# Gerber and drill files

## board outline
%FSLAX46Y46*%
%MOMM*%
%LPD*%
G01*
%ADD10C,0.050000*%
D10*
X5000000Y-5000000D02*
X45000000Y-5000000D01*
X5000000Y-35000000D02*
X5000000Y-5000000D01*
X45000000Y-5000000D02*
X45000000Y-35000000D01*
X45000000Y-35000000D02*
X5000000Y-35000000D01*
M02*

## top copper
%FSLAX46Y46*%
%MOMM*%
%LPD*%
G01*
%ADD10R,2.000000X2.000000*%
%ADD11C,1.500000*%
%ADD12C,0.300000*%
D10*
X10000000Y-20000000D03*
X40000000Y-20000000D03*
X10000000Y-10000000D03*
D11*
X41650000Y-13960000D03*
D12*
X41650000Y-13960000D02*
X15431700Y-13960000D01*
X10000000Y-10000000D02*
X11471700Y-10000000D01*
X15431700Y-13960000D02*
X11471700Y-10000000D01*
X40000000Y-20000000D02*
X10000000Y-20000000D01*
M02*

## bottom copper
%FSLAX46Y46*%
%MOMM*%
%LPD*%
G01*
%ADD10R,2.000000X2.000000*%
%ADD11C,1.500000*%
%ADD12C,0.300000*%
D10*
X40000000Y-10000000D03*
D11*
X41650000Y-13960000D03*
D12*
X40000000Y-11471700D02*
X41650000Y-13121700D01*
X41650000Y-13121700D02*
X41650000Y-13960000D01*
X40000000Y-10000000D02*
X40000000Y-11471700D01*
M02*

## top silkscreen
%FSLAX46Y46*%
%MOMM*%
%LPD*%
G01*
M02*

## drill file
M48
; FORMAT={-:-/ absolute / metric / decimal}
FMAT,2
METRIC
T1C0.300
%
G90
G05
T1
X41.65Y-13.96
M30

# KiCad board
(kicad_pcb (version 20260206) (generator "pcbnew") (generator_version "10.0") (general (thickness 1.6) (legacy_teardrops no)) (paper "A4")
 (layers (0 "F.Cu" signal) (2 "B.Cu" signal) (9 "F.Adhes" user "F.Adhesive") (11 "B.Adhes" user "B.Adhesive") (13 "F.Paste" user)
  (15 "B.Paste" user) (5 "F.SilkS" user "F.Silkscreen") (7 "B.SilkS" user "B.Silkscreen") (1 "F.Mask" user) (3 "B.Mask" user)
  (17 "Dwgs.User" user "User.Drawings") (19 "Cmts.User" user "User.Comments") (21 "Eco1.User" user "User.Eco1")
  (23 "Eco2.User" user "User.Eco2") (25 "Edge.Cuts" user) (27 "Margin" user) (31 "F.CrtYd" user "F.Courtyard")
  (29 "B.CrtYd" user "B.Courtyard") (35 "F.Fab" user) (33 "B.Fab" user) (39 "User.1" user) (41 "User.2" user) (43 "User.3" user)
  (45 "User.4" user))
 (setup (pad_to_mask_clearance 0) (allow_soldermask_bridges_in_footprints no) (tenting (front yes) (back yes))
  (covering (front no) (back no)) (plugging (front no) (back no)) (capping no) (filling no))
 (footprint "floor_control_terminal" (layer "F.Cu") (at 10 20)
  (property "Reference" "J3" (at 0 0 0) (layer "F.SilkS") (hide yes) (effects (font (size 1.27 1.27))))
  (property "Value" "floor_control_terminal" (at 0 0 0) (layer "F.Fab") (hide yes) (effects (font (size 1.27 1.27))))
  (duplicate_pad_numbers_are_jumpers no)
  (pad "1" smd rect (at 0 0) (size 2 2) (layers "F.Cu" "F.Mask" "F.Paste") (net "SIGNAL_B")))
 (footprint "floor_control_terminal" (layer "F.Cu") (at 40 20)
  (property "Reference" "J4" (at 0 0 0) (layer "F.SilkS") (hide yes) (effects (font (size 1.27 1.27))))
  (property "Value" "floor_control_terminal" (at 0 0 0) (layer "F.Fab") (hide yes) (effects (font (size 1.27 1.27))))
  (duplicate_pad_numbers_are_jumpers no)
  (pad "1" smd rect (at 0 0) (size 2 2) (layers "F.Cu" "F.Mask" "F.Paste") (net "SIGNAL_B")))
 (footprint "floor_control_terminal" (layer "F.Cu") (at 10 10)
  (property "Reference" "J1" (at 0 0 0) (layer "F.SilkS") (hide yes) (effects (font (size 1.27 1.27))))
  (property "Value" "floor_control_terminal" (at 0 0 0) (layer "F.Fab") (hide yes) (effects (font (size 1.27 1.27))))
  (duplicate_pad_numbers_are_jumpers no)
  (pad "1" smd rect (at 0 0) (size 2 2) (layers "F.Cu" "F.Mask" "F.Paste") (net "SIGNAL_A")))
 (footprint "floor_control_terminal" (layer "B.Cu") (at 40 10)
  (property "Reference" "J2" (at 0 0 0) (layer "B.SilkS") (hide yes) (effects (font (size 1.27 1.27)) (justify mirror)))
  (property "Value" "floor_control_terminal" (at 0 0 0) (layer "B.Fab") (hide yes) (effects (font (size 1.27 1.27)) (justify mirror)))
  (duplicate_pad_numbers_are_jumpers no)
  (pad "1" smd rect (at 0 0) (size 2 2) (layers "B.Cu" "B.Mask" "B.Paste") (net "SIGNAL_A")))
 (gr_line (start 5 5) (end 45 5) (stroke (width 0.05) (type default)) (layer "Edge.Cuts"))
 (gr_line (start 5 35) (end 5 5) (stroke (width 0.05) (type default)) (layer "Edge.Cuts"))
 (gr_line (start 45 5) (end 45 35) (stroke (width 0.05) (type default)) (layer "Edge.Cuts"))
 (gr_line (start 45 35) (end 5 35) (stroke (width 0.05) (type default)) (layer "Edge.Cuts"))
 (segment (start 41.65 13.96) (end 15.4317 13.96) (width 0.3) (layer "F.Cu") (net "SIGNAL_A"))
 (segment (start 10 10) (end 11.4717 10) (width 0.3) (layer "F.Cu") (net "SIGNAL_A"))
 (segment (start 15.4317 13.96) (end 11.4717 10) (width 0.3) (layer "F.Cu") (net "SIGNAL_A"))
 (via (at 41.65 13.96) (size 1.5) (drill 0.3) (layers "F.Cu" "B.Cu") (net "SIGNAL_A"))
 (segment (start 40 11.4717) (end 41.65 13.1217) (width 0.3) (layer "B.Cu") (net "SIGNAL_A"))
 (segment (start 41.65 13.1217) (end 41.65 13.96) (width 0.3) (layer "B.Cu") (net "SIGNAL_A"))
 (segment (start 40 10) (end 40 11.4717) (width 0.3) (layer "B.Cu") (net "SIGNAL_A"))
 (segment (start 40 20) (end 10 20) (width 0.3) (layer "F.Cu") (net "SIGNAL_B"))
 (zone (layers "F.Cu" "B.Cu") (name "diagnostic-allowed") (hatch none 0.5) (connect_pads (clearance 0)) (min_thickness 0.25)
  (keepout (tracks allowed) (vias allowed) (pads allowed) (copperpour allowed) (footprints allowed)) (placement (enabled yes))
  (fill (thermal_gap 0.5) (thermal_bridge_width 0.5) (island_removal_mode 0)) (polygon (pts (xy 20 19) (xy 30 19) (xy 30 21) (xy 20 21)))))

